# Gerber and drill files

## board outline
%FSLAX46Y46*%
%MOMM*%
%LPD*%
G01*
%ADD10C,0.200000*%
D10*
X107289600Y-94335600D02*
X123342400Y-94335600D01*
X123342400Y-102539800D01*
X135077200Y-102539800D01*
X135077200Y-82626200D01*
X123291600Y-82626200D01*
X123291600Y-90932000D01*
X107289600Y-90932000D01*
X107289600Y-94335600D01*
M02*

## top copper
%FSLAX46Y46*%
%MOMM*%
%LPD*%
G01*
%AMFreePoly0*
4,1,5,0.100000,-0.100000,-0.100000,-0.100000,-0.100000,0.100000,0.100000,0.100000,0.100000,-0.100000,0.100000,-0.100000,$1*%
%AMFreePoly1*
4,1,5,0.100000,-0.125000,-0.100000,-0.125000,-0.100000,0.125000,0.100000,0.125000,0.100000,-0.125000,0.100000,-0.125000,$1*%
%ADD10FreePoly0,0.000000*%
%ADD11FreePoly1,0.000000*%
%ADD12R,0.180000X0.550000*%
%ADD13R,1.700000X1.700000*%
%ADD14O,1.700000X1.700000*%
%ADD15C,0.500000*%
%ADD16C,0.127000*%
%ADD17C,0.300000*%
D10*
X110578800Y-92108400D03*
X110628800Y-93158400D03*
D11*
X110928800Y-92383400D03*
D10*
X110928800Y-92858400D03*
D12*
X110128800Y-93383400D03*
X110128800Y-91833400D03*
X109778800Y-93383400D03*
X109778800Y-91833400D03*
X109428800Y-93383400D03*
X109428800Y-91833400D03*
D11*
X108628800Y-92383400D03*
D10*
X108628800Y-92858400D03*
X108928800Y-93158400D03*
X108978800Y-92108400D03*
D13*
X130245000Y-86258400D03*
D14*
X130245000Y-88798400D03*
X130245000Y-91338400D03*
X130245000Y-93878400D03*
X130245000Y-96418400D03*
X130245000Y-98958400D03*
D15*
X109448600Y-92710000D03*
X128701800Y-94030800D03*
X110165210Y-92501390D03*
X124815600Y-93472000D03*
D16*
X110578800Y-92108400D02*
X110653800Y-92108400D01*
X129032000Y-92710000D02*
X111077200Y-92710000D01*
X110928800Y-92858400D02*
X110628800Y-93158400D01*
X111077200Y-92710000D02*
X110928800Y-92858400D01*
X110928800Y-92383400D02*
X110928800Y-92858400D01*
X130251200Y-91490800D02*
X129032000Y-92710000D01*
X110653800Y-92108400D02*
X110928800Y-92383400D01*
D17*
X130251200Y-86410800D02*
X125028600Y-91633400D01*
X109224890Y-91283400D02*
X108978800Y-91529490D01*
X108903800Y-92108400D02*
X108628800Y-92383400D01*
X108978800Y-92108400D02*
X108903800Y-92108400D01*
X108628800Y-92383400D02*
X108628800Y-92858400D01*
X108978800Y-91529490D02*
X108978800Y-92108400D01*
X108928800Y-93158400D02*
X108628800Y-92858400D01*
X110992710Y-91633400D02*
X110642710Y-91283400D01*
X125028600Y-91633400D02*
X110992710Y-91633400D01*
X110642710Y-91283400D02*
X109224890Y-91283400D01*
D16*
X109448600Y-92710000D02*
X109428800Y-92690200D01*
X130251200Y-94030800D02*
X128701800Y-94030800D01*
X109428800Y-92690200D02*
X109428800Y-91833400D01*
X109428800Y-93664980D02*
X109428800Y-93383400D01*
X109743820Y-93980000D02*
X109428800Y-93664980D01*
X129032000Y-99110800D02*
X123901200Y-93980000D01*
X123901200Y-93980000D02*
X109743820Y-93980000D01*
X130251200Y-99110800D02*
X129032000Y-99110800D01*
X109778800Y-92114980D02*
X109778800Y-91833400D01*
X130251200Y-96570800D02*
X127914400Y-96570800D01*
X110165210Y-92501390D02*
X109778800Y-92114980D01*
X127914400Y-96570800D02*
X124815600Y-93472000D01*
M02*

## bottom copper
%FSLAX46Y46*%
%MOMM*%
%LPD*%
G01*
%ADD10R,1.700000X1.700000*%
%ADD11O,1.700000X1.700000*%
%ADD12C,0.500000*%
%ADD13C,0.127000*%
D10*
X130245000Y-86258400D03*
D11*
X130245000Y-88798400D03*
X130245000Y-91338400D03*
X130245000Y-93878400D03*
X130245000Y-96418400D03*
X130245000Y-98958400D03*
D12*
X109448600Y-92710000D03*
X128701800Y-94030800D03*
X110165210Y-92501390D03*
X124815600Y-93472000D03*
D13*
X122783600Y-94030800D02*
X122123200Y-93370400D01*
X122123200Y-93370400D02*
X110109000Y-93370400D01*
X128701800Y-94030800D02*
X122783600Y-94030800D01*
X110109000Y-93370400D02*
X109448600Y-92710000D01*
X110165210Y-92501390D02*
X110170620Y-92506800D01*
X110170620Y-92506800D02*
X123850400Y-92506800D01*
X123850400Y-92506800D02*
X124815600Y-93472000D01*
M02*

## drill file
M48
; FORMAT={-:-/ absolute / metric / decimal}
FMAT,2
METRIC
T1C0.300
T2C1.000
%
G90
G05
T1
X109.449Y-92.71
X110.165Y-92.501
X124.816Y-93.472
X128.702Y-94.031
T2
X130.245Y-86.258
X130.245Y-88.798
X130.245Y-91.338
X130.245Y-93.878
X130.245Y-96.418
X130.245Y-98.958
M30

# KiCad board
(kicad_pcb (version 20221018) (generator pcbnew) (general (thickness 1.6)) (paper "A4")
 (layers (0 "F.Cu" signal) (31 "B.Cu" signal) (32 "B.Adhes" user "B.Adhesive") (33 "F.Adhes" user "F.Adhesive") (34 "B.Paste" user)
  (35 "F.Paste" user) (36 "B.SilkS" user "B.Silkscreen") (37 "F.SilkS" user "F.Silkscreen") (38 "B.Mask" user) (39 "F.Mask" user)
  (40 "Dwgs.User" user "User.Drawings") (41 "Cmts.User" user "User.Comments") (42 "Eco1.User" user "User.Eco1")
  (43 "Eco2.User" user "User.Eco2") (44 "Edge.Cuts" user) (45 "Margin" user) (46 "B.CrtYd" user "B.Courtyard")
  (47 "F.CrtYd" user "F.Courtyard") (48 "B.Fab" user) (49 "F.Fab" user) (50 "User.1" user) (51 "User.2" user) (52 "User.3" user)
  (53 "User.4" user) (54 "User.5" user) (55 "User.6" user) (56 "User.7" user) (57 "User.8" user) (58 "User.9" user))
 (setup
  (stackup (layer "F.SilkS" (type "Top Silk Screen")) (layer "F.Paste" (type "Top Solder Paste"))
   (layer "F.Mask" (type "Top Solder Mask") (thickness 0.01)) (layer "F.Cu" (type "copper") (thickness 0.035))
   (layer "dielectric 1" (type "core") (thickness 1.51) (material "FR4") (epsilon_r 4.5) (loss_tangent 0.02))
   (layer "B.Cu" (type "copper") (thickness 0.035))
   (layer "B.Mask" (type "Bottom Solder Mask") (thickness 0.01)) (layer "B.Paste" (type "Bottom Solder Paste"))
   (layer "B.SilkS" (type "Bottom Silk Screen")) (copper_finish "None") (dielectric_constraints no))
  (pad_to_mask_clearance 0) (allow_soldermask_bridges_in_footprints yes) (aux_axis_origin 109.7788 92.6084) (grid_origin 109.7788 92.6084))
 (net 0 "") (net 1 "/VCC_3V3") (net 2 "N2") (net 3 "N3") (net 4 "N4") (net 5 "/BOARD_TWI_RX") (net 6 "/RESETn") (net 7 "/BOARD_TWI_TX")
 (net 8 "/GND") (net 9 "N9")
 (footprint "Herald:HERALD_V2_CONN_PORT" (layer "F.Cu") (at 109.7788 92.6084)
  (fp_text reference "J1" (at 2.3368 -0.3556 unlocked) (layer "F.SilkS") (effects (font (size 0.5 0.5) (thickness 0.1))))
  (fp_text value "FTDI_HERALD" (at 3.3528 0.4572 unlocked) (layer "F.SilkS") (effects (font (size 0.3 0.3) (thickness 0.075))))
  (pad "1" smd custom (at 0.8 -0.5) (size 0.2 0.2) (layers "F.Cu" "F.Paste" "F.Mask") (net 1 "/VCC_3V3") (thermal_bridge_angle 45)
   (options (clearance outline) (anchor rect)) (primitives))
  (pad "1" smd custom (at 0.85 0.55) (size 0.2 0.2) (layers "F.Cu" "F.Paste" "F.Mask") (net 1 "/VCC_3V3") (thermal_bridge_angle 45)
   (options (clearance outline) (anchor rect)) (primitives))
  (pad "1" smd custom (at 1.15 -0.225) (size 0.2 0.25) (layers "F.Cu" "F.Paste" "F.Mask") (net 1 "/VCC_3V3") (thermal_bridge_angle 45)
   (options (clearance outline) (anchor rect)) (primitives))
  (pad "1" smd custom (at 1.15 0.25) (size 0.2 0.2) (layers "F.Cu" "F.Paste" "F.Mask") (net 1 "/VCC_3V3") (thermal_bridge_angle 45)
   (options (clearance outline) (anchor rect)) (primitives))
  (pad "2" smd rect (at 0.35 0.775) (size 0.18 0.55) (layers "F.Cu" "F.Paste" "F.Mask") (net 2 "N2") (thermal_bridge_angle 45))
  (pad "3" smd rect (at 0.35 -0.775) (size 0.18 0.55) (layers "F.Cu" "F.Paste" "F.Mask") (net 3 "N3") (thermal_bridge_angle 45))
  (pad "4" smd rect (at 0 0.775) (size 0.18 0.55) (layers "F.Cu" "F.Paste" "F.Mask") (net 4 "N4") (thermal_bridge_angle 45))
  (pad "5" smd rect (at 0 -0.775) (size 0.18 0.55) (layers "F.Cu" "F.Paste" "F.Mask") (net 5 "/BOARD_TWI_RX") (thermal_bridge_angle 45))
  (pad "6" smd rect (at -0.35 0.775) (size 0.18 0.55) (layers "F.Cu" "F.Paste" "F.Mask") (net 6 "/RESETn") (thermal_bridge_angle 45))
  (pad "7" smd rect (at -0.35 -0.775) (size 0.18 0.55) (layers "F.Cu" "F.Paste" "F.Mask") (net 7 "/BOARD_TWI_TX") (thermal_bridge_angle 45))
  (pad "8" smd custom (at -1.15 -0.225) (size 0.2 0.25) (layers "F.Cu" "F.Paste" "F.Mask") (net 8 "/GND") (thermal_bridge_angle 45)
   (options (clearance outline) (anchor rect)) (primitives))
  (pad "8" smd custom (at -1.15 0.25) (size 0.2 0.2) (layers "F.Cu" "F.Paste" "F.Mask") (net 8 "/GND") (thermal_bridge_angle 45)
   (options (clearance outline) (anchor rect)) (primitives))
  (pad "8" smd custom (at -0.85 0.55) (size 0.2 0.2) (layers "F.Cu" "F.Paste" "F.Mask") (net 8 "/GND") (thermal_bridge_angle 45)
   (options (clearance outline) (anchor rect)) (primitives))
  (pad "8" smd custom (at -0.8 -0.5) (size 0.2 0.2) (layers "F.Cu" "F.Paste" "F.Mask") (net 8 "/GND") (thermal_bridge_angle 45)
   (options (clearance outline) (anchor rect)) (primitives)))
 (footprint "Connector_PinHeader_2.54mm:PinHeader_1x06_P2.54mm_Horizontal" (layer "F.Cu") (at 130.245 86.2584)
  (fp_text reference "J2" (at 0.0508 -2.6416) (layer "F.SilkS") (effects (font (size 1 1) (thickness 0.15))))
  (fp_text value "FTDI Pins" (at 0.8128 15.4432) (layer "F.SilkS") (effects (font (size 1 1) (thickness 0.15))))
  (pad "1" thru_hole rect (at 0 0) (size 1.7 1.7) (drill 1) (layers "*.Cu" "*.Mask") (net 8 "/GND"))
  (pad "2" thru_hole oval (at 0 2.54) (size 1.7 1.7) (drill 1) (layers "*.Cu" "*.Mask") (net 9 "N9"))
  (pad "3" thru_hole oval (at 0 5.08) (size 1.7 1.7) (drill 1) (layers "*.Cu" "*.Mask") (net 1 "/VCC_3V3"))
  (pad "4" thru_hole oval (at 0 7.62) (size 1.7 1.7) (drill 1) (layers "*.Cu" "*.Mask") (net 7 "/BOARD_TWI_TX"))
  (pad "5" thru_hole oval (at 0 10.16) (size 1.7 1.7) (drill 1) (layers "*.Cu" "*.Mask") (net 5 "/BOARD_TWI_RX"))
  (pad "6" thru_hole oval (at 0 12.7) (size 1.7 1.7) (drill 1) (layers "*.Cu" "*.Mask") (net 6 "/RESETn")))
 (gr_poly
  (pts (xy 107.2896 94.3356) (xy 123.3424 94.3356) (xy 123.3424 102.5398) (xy 135.0772 102.5398) (xy 135.0772 82.6262) (xy 123.2916 82.6262)
   (xy 123.2916 90.932) (xy 107.2896 90.932))
  (stroke (width 0.2) (type solid)) (fill none) (layer "Edge.Cuts"))
 (segment (start 110.5788 92.1084) (end 110.6538 92.1084) (width 0.127) (layer "F.Cu") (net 1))
 (segment (start 129.032 92.71) (end 111.0772 92.71) (width 0.127) (layer "F.Cu") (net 1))
 (segment (start 110.9288 92.8584) (end 110.6288 93.1584) (width 0.127) (layer "F.Cu") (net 1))
 (segment (start 111.0772 92.71) (end 110.9288 92.8584) (width 0.127) (layer "F.Cu") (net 1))
 (segment (start 110.9288 92.3834) (end 110.9288 92.8584) (width 0.127) (layer "F.Cu") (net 1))
 (segment (start 130.2512 91.4908) (end 129.032 92.71) (width 0.127) (layer "F.Cu") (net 1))
 (segment (start 110.6538 92.1084) (end 110.9288 92.3834) (width 0.127) (layer "F.Cu") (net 1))
 (segment (start 130.2512 86.4108) (end 125.0286 91.6334) (width 0.3) (layer "F.Cu") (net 8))
 (segment (start 109.22489 91.2834) (end 108.9788 91.52949) (width 0.3) (layer "F.Cu") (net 8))
 (segment (start 108.9038 92.1084) (end 108.6288 92.3834) (width 0.3) (layer "F.Cu") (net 8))
 (segment (start 108.9788 92.1084) (end 108.9038 92.1084) (width 0.3) (layer "F.Cu") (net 8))
 (segment (start 108.6288 92.3834) (end 108.6288 92.8584) (width 0.3) (layer "F.Cu") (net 8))
 (segment (start 108.9788 91.52949) (end 108.9788 92.1084) (width 0.3) (layer "F.Cu") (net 8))
 (segment (start 108.9288 93.1584) (end 108.6288 92.8584) (width 0.3) (layer "F.Cu") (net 8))
 (segment (start 110.99271 91.6334) (end 110.64271 91.2834) (width 0.3) (layer "F.Cu") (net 8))
 (segment (start 125.0286 91.6334) (end 110.99271 91.6334) (width 0.3) (layer "F.Cu") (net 8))
 (segment (start 110.64271 91.2834) (end 109.22489 91.2834) (width 0.3) (layer "F.Cu") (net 8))
 (segment (start 109.4486 92.71) (end 109.4288 92.6902) (width 0.127) (layer "F.Cu") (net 7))
 (segment (start 130.2512 94.0308) (end 128.7018 94.0308) (width 0.127) (layer "F.Cu") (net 7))
 (segment (start 109.4288 92.6902) (end 109.4288 91.8334) (width 0.127) (layer "F.Cu") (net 7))
 (via (at 109.4486 92.71) (size 0.5) (drill 0.3) (layers "F.Cu" "B.Cu") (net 7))
 (via (at 128.7018 94.0308) (size 0.5) (drill 0.3) (layers "F.Cu" "B.Cu") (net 7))
 (segment (start 122.7836 94.0308) (end 122.1232 93.3704) (width 0.127) (layer "B.Cu") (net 7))
 (segment (start 122.1232 93.3704) (end 110.109 93.3704) (width 0.127) (layer "B.Cu") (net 7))
 (segment (start 128.7018 94.0308) (end 122.7836 94.0308) (width 0.127) (layer "B.Cu") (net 7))
 (segment (start 110.109 93.3704) (end 109.4486 92.71) (width 0.127) (layer "B.Cu") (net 7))
 (segment (start 109.4288 93.66498) (end 109.4288 93.3834) (width 0.127) (layer "F.Cu") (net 6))
 (segment (start 109.74382 93.98) (end 109.4288 93.66498) (width 0.127) (layer "F.Cu") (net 6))
 (segment (start 129.032 99.1108) (end 123.9012 93.98) (width 0.127) (layer "F.Cu") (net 6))
 (segment (start 123.9012 93.98) (end 109.74382 93.98) (width 0.127) (layer "F.Cu") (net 6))
 (segment (start 130.2512 99.1108) (end 129.032 99.1108) (width 0.127) (layer "F.Cu") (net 6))
 (segment (start 109.7788 92.11498) (end 109.7788 91.8334) (width 0.127) (layer "F.Cu") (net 5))
 (segment (start 130.2512 96.5708) (end 127.9144 96.5708) (width 0.127) (layer "F.Cu") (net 5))
 (segment (start 110.16521 92.50139) (end 109.7788 92.11498) (width 0.127) (layer "F.Cu") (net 5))
 (segment (start 127.9144 96.5708) (end 124.8156 93.472) (width 0.127) (layer "F.Cu") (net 5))
 (via (at 110.16521 92.50139) (size 0.5) (drill 0.3) (layers "F.Cu" "B.Cu") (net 5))
 (via (at 124.8156 93.472) (size 0.5) (drill 0.3) (layers "F.Cu" "B.Cu") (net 5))
 (segment (start 110.16521 92.50139) (end 110.17062 92.5068) (width 0.127) (layer "B.Cu") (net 5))
 (segment (start 110.17062 92.5068) (end 123.8504 92.5068) (width 0.127) (layer "B.Cu") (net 5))
 (segment (start 123.8504 92.5068) (end 124.8156 93.472) (width 0.127) (layer "B.Cu") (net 5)))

